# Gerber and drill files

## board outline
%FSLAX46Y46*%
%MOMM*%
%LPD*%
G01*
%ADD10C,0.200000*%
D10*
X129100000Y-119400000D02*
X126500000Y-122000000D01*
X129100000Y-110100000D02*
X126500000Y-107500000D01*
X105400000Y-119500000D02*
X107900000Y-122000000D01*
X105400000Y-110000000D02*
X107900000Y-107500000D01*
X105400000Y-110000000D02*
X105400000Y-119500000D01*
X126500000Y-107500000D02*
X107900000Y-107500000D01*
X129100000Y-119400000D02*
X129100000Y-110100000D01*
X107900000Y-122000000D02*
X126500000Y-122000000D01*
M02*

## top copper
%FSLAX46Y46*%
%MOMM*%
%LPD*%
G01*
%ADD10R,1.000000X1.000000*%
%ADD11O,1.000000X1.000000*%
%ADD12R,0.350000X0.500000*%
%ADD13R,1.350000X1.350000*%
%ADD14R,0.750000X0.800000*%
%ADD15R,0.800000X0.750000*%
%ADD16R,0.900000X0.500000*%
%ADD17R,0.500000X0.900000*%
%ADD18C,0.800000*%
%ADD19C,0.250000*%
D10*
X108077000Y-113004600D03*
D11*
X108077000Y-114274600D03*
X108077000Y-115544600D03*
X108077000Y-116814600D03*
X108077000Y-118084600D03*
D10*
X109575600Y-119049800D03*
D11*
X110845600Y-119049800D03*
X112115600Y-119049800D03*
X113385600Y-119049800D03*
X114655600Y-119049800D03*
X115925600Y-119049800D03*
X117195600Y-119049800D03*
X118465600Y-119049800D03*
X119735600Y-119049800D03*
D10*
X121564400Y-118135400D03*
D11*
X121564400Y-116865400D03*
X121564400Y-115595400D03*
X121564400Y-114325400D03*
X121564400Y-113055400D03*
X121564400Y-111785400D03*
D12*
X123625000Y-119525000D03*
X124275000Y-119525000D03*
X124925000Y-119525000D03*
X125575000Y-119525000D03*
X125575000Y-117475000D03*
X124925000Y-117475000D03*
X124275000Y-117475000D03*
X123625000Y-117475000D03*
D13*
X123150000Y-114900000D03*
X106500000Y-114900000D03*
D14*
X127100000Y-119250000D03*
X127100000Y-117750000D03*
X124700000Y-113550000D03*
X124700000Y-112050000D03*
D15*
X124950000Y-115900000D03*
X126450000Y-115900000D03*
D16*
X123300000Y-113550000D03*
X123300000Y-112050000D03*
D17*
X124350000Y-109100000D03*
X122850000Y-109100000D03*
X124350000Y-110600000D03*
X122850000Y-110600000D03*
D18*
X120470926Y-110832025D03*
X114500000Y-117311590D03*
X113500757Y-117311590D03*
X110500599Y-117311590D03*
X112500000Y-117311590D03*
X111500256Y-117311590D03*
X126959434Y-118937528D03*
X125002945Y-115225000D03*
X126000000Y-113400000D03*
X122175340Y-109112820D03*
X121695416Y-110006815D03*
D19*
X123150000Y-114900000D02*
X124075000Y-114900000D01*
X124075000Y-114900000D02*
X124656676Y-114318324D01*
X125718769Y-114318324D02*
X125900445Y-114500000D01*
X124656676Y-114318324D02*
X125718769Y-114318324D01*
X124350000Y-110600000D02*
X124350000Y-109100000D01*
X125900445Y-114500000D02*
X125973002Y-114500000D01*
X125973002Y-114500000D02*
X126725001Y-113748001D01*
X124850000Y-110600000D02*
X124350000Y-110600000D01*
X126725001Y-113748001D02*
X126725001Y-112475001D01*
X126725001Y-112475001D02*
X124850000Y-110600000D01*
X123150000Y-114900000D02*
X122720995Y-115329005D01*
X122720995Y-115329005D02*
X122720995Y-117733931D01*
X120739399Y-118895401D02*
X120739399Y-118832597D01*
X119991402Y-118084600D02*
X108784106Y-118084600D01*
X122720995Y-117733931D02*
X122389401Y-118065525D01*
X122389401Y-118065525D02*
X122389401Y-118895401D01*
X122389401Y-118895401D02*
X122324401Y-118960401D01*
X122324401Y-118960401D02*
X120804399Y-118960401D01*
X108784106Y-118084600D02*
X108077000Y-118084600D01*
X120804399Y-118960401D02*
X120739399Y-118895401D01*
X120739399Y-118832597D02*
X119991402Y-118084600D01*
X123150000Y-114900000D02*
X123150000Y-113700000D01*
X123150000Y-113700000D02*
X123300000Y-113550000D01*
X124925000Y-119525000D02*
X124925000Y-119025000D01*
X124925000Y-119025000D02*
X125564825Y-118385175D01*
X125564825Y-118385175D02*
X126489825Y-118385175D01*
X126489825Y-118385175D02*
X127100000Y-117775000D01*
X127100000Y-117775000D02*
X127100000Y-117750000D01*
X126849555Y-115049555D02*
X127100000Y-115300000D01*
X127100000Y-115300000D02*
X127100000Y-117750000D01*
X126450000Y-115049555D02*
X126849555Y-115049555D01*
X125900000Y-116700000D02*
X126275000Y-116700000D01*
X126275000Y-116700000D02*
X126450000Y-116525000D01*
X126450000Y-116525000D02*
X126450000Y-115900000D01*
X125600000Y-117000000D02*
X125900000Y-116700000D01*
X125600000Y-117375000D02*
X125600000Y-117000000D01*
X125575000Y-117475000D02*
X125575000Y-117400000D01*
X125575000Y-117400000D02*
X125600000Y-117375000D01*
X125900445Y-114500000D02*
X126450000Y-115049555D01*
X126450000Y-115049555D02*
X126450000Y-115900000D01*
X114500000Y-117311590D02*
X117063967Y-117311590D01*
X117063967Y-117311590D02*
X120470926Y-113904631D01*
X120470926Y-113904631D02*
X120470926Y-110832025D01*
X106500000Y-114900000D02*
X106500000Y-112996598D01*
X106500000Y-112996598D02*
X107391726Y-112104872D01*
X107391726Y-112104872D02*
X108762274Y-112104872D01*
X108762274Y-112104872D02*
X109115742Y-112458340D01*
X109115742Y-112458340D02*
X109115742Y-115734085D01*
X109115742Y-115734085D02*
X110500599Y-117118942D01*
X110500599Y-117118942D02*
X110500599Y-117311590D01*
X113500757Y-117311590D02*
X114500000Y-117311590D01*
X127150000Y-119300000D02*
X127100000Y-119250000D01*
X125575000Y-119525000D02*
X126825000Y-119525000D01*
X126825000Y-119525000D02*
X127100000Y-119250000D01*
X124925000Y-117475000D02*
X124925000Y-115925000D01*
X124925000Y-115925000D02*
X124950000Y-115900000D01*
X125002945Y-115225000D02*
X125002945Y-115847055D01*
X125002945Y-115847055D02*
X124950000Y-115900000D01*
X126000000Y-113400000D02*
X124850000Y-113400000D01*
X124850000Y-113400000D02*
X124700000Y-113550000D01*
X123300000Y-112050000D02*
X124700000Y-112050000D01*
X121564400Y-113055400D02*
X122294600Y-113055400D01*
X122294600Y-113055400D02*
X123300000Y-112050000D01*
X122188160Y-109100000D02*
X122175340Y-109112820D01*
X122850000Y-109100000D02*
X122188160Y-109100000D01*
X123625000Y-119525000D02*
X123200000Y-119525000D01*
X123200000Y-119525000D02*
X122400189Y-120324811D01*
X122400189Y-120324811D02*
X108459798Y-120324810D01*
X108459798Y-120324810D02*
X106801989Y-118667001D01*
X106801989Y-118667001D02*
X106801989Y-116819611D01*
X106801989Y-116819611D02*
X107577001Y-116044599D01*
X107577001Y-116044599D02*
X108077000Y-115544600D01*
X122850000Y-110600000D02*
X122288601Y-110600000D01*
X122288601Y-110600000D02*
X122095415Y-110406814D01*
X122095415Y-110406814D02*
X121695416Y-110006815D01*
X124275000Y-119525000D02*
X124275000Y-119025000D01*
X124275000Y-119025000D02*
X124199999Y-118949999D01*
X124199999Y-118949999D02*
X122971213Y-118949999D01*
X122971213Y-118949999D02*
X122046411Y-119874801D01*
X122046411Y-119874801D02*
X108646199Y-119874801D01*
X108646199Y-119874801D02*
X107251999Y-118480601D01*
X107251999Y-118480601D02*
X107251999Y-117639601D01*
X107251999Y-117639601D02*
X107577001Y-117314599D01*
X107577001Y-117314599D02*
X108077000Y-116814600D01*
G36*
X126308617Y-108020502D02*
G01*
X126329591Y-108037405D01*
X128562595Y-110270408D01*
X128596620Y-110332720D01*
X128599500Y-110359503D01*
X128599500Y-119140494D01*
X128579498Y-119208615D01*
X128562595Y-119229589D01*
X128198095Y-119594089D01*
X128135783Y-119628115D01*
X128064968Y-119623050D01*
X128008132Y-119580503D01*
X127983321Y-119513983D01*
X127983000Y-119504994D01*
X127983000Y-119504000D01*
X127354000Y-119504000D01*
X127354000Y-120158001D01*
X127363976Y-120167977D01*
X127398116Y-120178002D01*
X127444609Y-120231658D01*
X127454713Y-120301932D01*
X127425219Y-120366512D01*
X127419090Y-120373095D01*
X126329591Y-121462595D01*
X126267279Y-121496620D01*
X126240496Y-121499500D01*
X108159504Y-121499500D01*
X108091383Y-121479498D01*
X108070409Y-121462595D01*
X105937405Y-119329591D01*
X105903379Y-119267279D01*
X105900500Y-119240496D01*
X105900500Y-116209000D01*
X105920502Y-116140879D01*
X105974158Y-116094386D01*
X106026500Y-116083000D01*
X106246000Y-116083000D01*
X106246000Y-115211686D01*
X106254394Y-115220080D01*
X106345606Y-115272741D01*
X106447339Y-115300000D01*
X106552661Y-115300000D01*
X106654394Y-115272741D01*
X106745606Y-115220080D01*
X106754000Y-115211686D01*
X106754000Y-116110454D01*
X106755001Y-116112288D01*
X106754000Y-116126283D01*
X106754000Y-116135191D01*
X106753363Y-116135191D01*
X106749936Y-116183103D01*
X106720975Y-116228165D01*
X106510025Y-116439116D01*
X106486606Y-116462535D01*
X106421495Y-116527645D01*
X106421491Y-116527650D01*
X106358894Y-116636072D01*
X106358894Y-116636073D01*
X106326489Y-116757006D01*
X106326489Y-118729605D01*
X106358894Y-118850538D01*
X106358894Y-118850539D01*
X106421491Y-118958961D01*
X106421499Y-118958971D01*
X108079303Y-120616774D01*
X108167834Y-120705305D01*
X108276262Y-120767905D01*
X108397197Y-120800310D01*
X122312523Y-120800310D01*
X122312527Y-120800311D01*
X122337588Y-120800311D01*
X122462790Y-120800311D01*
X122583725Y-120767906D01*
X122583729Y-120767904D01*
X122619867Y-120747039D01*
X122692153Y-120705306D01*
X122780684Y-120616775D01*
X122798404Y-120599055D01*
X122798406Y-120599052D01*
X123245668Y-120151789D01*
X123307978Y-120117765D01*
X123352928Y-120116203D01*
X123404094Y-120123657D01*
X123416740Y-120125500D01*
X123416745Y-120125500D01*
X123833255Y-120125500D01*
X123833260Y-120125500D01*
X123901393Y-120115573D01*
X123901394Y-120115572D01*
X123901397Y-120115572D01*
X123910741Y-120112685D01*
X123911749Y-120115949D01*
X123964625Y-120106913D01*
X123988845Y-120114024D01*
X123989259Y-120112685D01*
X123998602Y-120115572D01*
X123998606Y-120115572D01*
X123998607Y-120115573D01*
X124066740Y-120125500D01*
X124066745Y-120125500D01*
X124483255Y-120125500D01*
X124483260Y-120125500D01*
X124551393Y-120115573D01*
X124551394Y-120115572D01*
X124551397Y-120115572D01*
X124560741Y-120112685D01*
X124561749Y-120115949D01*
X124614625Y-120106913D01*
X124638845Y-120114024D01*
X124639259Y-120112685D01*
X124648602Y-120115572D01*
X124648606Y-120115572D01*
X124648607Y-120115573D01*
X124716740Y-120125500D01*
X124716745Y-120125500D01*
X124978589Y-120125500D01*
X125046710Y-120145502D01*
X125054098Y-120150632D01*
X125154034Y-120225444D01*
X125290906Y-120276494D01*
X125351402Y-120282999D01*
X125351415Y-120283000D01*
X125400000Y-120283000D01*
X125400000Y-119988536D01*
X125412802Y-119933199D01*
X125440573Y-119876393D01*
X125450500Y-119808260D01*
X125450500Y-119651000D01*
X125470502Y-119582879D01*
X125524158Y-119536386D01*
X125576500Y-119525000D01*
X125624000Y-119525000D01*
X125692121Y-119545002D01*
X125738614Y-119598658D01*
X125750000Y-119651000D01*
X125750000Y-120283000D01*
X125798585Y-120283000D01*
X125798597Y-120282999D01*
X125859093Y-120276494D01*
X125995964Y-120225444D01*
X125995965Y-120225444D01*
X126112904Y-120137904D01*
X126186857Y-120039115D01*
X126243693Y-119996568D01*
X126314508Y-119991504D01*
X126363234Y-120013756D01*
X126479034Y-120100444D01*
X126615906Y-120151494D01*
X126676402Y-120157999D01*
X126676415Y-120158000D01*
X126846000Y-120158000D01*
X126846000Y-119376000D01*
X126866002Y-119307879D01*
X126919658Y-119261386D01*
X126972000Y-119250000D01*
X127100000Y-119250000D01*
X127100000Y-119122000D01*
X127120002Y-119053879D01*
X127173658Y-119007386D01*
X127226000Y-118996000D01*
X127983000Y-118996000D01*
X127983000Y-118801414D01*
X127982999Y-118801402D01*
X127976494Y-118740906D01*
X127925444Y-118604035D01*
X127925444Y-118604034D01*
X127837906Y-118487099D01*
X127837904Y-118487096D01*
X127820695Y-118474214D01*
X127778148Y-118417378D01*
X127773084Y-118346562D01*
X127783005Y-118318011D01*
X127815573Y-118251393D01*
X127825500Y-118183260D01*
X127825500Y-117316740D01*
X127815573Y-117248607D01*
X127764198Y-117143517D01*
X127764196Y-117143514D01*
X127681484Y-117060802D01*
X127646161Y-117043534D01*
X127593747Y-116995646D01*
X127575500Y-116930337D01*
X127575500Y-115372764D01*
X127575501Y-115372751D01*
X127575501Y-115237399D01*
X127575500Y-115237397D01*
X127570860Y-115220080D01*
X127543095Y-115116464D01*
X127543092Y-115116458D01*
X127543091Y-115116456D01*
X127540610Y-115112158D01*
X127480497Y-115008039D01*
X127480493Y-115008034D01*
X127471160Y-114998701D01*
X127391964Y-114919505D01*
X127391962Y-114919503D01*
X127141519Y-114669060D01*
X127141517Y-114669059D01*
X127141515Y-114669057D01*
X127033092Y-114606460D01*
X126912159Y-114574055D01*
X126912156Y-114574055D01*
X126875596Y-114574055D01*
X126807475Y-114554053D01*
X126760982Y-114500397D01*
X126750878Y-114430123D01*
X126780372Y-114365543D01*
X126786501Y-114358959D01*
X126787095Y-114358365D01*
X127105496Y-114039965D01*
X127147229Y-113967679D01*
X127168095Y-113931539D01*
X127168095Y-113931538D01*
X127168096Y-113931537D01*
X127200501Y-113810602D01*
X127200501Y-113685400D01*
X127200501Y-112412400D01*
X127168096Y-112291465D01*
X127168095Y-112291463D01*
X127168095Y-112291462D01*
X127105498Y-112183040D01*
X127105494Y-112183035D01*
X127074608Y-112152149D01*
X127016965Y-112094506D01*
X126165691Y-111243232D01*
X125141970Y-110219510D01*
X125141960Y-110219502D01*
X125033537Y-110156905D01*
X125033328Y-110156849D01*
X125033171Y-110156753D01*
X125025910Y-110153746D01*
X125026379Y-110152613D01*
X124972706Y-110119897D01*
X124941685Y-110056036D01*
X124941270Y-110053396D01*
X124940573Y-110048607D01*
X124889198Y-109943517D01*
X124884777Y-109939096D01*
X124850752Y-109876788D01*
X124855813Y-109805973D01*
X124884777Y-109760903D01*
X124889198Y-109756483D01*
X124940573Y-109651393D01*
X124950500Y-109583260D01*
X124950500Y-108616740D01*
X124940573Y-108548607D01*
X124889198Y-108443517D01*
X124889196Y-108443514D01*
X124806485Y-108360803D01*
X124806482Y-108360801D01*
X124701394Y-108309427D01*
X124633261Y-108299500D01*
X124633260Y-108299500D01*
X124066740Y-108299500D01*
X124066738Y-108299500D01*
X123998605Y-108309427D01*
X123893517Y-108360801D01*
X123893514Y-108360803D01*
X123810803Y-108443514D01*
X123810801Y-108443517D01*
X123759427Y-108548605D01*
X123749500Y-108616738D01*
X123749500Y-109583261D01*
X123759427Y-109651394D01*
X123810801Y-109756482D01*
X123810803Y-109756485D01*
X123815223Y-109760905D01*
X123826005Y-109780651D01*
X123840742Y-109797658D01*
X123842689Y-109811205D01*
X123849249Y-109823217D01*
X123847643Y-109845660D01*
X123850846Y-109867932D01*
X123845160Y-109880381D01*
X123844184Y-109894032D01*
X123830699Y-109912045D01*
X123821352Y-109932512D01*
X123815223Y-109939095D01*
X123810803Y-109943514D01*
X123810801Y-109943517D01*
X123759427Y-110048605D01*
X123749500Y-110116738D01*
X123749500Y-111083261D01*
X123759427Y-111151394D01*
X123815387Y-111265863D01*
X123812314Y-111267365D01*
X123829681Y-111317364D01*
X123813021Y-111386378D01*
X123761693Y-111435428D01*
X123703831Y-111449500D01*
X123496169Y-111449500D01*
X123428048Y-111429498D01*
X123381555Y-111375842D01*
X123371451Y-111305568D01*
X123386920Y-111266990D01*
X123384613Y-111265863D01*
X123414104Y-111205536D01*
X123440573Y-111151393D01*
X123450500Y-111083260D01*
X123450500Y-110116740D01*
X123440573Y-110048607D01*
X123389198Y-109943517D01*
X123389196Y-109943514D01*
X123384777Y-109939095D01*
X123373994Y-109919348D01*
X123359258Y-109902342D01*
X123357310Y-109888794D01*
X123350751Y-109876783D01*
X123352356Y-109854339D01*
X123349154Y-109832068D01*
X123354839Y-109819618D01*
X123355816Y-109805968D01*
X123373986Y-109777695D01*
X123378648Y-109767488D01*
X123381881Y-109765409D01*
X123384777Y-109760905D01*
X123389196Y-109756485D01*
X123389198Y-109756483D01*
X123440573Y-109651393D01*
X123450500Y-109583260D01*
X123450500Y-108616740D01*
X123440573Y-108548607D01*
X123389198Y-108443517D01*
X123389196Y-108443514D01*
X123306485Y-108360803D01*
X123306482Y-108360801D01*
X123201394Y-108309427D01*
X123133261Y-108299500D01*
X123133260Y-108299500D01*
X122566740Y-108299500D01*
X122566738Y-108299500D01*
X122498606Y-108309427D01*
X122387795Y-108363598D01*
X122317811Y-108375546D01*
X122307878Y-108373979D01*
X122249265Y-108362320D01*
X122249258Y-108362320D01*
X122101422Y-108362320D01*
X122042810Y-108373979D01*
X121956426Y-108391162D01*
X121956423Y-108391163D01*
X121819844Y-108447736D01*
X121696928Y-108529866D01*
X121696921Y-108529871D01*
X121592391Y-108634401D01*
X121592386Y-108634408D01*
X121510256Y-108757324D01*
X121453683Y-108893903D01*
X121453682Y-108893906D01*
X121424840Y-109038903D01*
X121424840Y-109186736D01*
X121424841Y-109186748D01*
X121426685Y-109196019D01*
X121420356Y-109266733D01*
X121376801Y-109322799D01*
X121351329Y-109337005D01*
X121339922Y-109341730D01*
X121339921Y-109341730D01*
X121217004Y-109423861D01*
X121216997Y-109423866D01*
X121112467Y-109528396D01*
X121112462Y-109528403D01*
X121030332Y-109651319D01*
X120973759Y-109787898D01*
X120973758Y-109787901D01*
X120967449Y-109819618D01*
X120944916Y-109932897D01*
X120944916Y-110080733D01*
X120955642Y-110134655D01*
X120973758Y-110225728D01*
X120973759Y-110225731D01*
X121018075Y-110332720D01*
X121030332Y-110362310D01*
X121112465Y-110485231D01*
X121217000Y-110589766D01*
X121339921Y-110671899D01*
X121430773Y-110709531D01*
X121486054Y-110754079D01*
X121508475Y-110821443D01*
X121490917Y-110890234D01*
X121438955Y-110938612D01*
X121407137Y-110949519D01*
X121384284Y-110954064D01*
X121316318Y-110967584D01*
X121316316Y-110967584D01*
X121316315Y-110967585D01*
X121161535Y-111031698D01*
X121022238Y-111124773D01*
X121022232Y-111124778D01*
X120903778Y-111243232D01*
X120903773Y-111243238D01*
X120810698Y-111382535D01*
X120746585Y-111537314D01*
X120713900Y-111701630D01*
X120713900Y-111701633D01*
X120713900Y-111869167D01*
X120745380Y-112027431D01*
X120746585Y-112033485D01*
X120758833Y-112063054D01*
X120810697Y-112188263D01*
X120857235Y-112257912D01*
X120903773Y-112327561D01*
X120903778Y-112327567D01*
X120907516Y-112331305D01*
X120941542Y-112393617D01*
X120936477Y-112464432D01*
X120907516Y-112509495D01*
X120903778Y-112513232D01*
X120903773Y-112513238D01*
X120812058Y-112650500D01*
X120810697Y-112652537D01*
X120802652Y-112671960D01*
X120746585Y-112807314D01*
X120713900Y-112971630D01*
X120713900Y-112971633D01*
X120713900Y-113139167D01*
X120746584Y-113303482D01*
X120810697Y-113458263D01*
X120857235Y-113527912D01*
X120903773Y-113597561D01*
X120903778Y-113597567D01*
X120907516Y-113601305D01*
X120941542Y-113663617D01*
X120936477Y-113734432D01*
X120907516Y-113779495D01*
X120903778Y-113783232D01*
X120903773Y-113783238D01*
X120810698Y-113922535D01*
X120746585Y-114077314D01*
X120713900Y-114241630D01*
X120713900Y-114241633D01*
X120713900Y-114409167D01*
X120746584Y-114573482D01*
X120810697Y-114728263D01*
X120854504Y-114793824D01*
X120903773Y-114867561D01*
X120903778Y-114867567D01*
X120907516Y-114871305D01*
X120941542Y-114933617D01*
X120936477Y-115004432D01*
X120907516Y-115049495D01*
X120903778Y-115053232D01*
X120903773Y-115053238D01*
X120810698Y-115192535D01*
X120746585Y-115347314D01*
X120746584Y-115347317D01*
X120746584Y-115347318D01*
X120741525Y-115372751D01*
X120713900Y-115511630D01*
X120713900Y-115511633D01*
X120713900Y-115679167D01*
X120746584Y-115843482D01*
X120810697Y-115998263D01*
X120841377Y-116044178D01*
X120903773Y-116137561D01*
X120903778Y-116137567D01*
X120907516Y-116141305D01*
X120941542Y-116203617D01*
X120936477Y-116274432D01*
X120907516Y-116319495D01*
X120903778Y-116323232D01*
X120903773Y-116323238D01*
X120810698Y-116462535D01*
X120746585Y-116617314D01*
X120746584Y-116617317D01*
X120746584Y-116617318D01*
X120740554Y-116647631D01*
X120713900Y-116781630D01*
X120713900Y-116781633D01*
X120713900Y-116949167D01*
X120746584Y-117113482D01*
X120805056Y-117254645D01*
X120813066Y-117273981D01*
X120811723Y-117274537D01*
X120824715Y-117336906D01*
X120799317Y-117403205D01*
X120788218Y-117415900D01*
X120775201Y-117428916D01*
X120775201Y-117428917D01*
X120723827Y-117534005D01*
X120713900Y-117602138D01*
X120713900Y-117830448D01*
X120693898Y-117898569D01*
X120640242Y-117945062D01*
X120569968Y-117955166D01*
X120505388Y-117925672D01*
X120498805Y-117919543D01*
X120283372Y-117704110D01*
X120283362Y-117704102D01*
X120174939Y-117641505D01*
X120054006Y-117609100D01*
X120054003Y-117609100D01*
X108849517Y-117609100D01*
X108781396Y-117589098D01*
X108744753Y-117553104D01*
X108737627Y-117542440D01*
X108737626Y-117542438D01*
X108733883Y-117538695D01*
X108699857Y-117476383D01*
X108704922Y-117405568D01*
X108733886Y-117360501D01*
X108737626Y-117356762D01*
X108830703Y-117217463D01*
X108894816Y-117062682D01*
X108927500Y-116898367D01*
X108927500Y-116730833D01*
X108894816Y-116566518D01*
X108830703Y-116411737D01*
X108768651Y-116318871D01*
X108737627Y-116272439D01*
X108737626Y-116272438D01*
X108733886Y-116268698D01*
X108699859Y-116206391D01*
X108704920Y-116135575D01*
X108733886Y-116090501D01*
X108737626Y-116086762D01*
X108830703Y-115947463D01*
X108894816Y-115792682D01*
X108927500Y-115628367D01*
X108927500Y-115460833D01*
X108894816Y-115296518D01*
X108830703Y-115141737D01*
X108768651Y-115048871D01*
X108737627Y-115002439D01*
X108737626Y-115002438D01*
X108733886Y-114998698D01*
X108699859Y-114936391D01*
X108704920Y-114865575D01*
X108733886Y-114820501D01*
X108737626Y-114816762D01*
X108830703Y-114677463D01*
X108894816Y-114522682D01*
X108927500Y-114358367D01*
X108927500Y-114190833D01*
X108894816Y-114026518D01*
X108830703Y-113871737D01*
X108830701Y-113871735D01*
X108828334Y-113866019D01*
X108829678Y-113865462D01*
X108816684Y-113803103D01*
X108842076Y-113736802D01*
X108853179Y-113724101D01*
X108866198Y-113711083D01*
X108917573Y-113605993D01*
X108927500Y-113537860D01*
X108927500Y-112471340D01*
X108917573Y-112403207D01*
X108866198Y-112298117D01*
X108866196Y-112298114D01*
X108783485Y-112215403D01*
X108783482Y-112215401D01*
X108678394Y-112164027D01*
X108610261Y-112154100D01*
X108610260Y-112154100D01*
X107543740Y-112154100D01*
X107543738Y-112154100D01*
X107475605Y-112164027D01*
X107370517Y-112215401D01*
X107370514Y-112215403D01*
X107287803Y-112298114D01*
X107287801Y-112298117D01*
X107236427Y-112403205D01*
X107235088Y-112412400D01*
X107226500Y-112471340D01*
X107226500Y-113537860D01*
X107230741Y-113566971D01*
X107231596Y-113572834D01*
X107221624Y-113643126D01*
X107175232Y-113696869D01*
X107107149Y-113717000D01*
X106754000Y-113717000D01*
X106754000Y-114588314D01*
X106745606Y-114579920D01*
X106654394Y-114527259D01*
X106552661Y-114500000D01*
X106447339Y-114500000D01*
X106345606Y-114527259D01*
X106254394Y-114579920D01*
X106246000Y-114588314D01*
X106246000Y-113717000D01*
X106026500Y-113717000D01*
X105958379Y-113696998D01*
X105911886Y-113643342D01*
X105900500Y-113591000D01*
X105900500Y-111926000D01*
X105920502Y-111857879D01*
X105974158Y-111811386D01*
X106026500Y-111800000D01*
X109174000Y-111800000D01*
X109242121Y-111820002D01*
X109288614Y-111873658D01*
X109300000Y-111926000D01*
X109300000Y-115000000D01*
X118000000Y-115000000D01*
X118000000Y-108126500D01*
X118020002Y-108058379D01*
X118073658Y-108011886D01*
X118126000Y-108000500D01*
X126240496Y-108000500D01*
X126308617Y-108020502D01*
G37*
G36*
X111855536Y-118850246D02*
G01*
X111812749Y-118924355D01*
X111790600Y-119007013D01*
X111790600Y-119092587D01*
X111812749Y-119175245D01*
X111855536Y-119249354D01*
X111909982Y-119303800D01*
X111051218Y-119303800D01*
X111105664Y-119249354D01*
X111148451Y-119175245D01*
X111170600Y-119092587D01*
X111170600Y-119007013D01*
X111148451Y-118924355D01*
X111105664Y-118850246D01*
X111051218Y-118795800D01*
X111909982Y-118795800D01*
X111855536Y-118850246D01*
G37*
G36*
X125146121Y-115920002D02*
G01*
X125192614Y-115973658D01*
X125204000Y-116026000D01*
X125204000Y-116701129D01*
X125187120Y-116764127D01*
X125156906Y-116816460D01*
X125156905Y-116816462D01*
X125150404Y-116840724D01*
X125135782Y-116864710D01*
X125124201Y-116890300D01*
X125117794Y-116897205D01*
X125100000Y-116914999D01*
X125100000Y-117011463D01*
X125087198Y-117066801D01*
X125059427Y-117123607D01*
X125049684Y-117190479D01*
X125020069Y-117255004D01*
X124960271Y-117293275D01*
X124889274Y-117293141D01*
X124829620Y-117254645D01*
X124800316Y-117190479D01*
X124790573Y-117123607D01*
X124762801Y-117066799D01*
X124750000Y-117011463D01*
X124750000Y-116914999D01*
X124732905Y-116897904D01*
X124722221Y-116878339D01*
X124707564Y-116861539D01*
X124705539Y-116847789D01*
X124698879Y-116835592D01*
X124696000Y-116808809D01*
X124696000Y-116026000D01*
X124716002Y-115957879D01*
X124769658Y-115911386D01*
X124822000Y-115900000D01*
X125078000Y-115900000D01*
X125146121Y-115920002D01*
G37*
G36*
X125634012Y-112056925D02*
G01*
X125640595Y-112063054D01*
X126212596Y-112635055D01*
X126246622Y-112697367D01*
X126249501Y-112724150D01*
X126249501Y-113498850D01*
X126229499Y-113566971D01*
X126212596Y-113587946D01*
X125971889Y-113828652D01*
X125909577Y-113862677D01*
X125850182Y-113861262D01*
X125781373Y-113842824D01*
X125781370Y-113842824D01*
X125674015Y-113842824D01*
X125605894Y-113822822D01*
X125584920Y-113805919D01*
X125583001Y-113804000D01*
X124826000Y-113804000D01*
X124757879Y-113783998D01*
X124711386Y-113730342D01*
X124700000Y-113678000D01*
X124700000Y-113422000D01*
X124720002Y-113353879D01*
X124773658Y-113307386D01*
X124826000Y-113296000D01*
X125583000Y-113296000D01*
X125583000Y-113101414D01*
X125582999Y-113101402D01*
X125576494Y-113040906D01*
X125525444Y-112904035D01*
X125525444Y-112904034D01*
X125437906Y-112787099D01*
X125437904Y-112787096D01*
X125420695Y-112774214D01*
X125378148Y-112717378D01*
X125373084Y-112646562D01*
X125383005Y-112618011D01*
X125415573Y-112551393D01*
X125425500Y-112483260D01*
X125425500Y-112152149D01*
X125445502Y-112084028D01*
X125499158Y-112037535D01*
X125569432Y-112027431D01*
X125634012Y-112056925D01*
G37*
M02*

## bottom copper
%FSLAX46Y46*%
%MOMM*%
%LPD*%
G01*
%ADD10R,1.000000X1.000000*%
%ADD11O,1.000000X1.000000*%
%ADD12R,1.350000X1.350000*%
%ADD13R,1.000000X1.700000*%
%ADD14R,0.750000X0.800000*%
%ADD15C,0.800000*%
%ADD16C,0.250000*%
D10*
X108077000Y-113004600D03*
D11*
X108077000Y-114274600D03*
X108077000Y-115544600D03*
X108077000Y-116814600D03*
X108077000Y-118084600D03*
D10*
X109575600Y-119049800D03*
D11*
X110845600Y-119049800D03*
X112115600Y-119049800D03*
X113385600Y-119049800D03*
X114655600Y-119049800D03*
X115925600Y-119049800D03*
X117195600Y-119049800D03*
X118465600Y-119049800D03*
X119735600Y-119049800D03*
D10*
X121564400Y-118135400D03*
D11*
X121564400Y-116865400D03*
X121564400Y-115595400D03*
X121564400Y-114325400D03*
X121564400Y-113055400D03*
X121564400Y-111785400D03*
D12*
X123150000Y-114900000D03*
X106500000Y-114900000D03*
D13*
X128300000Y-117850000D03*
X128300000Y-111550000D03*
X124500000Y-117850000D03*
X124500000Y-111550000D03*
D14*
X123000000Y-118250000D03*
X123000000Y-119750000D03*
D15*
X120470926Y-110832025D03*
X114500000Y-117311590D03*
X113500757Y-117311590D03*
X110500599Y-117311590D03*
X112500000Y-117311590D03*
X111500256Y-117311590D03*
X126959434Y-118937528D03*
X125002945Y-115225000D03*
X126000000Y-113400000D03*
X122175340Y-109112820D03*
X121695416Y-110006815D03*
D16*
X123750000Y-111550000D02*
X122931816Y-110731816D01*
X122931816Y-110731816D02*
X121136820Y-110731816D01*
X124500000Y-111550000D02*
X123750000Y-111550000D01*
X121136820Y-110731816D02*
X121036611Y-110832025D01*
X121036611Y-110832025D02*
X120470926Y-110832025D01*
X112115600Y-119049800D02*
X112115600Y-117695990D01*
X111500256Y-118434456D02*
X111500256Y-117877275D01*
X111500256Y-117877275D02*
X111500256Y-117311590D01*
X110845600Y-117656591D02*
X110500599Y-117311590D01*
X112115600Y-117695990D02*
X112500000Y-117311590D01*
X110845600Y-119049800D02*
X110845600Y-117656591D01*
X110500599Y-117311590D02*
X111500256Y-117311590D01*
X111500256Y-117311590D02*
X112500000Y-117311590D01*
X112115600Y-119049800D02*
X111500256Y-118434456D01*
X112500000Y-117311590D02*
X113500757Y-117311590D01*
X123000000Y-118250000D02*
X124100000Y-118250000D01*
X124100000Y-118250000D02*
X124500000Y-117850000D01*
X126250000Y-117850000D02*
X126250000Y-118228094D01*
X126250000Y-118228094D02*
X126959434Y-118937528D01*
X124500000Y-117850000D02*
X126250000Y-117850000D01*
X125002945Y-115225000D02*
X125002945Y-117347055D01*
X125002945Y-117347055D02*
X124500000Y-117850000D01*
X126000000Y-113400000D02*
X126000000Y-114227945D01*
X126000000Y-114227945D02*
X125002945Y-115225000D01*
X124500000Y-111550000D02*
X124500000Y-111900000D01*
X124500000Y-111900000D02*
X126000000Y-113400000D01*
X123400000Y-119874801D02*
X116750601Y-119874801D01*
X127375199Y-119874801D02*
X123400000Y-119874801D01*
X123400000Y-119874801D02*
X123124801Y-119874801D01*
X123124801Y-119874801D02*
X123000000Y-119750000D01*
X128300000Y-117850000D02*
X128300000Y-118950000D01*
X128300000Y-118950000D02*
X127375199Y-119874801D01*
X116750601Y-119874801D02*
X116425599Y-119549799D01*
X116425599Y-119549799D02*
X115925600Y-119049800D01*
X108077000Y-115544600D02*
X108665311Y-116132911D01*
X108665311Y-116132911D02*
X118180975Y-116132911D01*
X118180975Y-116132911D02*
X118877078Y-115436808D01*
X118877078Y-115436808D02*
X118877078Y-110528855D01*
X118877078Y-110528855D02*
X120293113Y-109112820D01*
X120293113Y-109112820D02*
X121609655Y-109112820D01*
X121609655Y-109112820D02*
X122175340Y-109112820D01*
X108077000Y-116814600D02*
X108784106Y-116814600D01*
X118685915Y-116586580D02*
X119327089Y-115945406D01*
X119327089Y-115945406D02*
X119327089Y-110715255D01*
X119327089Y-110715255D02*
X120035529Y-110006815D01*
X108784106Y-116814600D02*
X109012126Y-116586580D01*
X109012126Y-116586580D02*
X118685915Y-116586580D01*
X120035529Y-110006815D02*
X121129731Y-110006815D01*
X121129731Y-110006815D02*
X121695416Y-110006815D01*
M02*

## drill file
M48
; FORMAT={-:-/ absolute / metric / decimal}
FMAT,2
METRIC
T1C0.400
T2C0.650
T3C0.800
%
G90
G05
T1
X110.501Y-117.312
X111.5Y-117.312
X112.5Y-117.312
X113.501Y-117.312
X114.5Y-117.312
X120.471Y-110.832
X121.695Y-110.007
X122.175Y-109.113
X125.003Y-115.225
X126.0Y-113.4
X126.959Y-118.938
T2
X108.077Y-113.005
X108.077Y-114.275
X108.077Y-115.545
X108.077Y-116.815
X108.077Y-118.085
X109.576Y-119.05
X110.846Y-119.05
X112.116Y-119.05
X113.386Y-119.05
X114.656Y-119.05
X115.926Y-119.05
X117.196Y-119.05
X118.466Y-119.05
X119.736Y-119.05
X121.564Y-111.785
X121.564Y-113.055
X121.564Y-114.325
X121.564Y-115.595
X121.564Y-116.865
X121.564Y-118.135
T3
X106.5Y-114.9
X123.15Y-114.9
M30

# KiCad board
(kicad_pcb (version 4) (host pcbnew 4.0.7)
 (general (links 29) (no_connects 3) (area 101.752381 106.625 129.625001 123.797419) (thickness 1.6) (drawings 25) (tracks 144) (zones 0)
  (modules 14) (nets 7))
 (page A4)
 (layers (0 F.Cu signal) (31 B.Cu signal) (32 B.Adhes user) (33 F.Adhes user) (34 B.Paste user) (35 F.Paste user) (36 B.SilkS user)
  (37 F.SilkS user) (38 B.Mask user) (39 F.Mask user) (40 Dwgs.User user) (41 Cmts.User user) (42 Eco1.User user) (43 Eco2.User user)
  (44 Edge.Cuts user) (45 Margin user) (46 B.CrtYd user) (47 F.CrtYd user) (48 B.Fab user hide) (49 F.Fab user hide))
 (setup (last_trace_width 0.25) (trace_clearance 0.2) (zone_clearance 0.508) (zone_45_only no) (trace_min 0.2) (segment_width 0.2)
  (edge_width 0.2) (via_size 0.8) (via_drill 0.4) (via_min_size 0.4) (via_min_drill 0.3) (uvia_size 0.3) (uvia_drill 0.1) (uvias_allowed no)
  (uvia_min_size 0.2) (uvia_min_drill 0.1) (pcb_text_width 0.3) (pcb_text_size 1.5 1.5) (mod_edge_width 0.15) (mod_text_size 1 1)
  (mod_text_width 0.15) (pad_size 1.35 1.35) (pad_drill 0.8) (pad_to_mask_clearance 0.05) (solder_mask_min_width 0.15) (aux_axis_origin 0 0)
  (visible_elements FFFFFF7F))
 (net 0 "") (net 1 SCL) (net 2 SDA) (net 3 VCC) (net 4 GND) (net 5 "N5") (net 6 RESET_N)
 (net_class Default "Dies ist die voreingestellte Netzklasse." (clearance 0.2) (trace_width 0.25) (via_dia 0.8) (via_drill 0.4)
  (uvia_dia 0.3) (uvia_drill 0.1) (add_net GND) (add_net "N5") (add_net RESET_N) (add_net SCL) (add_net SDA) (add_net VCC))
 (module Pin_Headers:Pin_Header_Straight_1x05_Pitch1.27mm (layer F.Cu) (at 108.077 113.0046)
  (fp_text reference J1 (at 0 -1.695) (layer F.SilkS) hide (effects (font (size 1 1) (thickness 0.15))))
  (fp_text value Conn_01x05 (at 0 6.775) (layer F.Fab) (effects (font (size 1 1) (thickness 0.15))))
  (pad 1 thru_hole rect (at 0 0) (size 1 1) (drill 0.65) (layers *.Cu *.Mask))
  (pad 2 thru_hole oval (at 0 1.27) (size 1 1) (drill 0.65) (layers *.Cu *.Mask))
  (pad 3 thru_hole oval (at 0 2.54) (size 1 1) (drill 0.65) (layers *.Cu *.Mask) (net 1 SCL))
  (pad 4 thru_hole oval (at 0 3.81) (size 1 1) (drill 0.65) (layers *.Cu *.Mask) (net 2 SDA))
  (pad 5 thru_hole oval (at 0 5.08) (size 1 1) (drill 0.65) (layers *.Cu *.Mask) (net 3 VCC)))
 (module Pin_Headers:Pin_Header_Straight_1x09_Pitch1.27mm (layer F.Cu) (at 109.5756 119.0498 90)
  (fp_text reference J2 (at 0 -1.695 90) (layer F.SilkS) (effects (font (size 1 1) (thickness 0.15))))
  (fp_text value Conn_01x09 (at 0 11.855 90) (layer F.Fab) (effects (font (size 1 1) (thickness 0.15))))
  (pad 1 thru_hole rect (at 0 0 90) (size 1 1) (drill 0.65) (layers *.Cu *.Mask))
  (pad 2 thru_hole oval (at 0 1.27 90) (size 1 1) (drill 0.65) (layers *.Cu *.Mask) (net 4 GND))
  (pad 3 thru_hole oval (at 0 2.54 90) (size 1 1) (drill 0.65) (layers *.Cu *.Mask) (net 4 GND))
  (pad 4 thru_hole oval (at 0 3.81 90) (size 1 1) (drill 0.65) (layers *.Cu *.Mask))
  (pad 5 thru_hole oval (at 0 5.08 90) (size 1 1) (drill 0.65) (layers *.Cu *.Mask))
  (pad 6 thru_hole oval (at 0 6.35 90) (size 1 1) (drill 0.65) (layers *.Cu *.Mask) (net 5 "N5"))
  (pad 7 thru_hole oval (at 0 7.62 90) (size 1 1) (drill 0.65) (layers *.Cu *.Mask))
  (pad 8 thru_hole oval (at 0 8.89 90) (size 1 1) (drill 0.65) (layers *.Cu *.Mask))
  (pad 9 thru_hole oval (at 0 10.16 90) (size 1 1) (drill 0.65) (layers *.Cu *.Mask)))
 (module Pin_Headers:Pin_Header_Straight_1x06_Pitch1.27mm (layer F.Cu) (at 121.5644 118.1354 180)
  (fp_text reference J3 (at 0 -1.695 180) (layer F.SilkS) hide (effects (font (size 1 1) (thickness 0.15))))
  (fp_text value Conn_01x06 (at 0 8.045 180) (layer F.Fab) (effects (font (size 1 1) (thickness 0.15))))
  (pad 1 thru_hole rect (at 0 0 180) (size 1 1) (drill 0.65) (layers *.Cu *.Mask))
  (pad 2 thru_hole oval (at 0 1.27 180) (size 1 1) (drill 0.65) (layers *.Cu *.Mask))
  (pad 3 thru_hole oval (at 0 2.54 180) (size 1 1) (drill 0.65) (layers *.Cu *.Mask))
  (pad 4 thru_hole oval (at 0 3.81 180) (size 1 1) (drill 0.65) (layers *.Cu *.Mask))
  (pad 5 thru_hole oval (at 0 5.08 180) (size 1 1) (drill 0.65) (layers *.Cu *.Mask) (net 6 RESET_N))
  (pad 6 thru_hole oval (at 0 6.35 180) (size 1 1) (drill 0.65) (layers *.Cu *.Mask)))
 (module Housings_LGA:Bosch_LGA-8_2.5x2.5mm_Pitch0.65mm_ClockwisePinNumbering (layer F.Cu) (at 124.6 118.5 180)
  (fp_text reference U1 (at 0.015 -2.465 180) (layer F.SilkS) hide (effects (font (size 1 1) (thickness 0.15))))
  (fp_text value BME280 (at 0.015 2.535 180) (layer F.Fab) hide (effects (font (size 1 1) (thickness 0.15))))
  (pad 4 smd rect (at 0.975 -1.025 270) (size 0.5 0.35) (layers F.Cu F.Paste F.Mask) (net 1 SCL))
  (pad 3 smd rect (at 0.325 -1.025 270) (size 0.5 0.35) (layers F.Cu F.Paste F.Mask) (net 2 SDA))
  (pad 2 smd rect (at -0.325 -1.025 270) (size 0.5 0.35) (layers F.Cu F.Paste F.Mask) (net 3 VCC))
  (pad 1 smd rect (at -0.975 -1.025 270) (size 0.5 0.35) (layers F.Cu F.Paste F.Mask) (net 4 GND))
  (pad 8 smd rect (at -0.975 1.025 270) (size 0.5 0.35) (layers F.Cu F.Paste F.Mask) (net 3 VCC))
  (pad 7 smd rect (at -0.325 1.025 270) (size 0.5 0.35) (layers F.Cu F.Paste F.Mask) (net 4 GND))
  (pad 6 smd rect (at 0.325 1.025 270) (size 0.5 0.35) (layers F.Cu F.Paste F.Mask) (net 3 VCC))
  (pad 5 smd rect (at 0.975 1.025 270) (size 0.5 0.35) (layers F.Cu F.Paste F.Mask) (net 3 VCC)))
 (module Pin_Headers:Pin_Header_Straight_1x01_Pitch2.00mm (layer F.Cu) (at 123.15 114.7)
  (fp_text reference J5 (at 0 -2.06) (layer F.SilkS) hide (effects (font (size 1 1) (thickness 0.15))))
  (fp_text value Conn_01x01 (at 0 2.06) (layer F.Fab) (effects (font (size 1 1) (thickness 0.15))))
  (pad 1 thru_hole rect (at 0 0.2) (size 1.35 1.35) (drill 0.8) (layers *.Cu *.Mask) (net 3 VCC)))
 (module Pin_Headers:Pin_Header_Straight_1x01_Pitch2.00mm (layer F.Cu) (at 106.5 114.8)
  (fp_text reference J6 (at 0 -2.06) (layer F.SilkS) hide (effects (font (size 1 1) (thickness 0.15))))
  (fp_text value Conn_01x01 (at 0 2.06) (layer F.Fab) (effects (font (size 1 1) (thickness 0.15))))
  (pad 1 thru_hole rect (at 0 0.1) (size 1.35 1.35) (drill 0.8) (layers *.Cu *.Mask) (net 4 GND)))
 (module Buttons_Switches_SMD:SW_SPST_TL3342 (layer B.Cu) (at 126.4 114.7 90)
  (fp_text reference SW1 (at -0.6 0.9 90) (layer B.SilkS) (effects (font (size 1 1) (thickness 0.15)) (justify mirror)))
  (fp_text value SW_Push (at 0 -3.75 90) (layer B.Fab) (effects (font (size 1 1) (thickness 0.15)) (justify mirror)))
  (pad 1 smd rect (at -3.15 1.9 90) (size 1.7 1) (layers B.Cu B.Paste B.Mask) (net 5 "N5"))
  (pad 1 smd rect (at 3.15 1.9 90) (size 1.7 1) (layers B.Cu B.Paste B.Mask) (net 5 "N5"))
  (pad 2 smd rect (at -3.15 -1.9 90) (size 1.7 1) (layers B.Cu B.Paste B.Mask) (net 4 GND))
  (pad 2 smd rect (at 3.15 -1.9 90) (size 1.7 1) (layers B.Cu B.Paste B.Mask) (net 4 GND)))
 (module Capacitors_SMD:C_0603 (layer F.Cu) (at 127.1 118.5 270)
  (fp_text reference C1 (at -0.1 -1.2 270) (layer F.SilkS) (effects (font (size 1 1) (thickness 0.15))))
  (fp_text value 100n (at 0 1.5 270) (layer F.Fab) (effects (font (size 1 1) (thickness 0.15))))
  (pad 2 smd rect (at 0.75 0 270) (size 0.8 0.75) (layers F.Cu F.Paste F.Mask) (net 4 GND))
  (pad 1 smd rect (at -0.75 0 270) (size 0.8 0.75) (layers F.Cu F.Paste F.Mask) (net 3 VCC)))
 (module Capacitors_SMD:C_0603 (layer F.Cu) (at 124.7 112.8 270)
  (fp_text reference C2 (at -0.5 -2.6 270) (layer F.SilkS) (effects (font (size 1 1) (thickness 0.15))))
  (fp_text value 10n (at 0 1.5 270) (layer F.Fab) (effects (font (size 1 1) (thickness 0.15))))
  (pad 2 smd rect (at 0.75 0 270) (size 0.8 0.75) (layers F.Cu F.Paste F.Mask) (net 4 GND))
  (pad 1 smd rect (at -0.75 0 270) (size 0.8 0.75) (layers F.Cu F.Paste F.Mask) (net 6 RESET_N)))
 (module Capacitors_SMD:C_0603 (layer F.Cu) (at 125.7 115.9 180)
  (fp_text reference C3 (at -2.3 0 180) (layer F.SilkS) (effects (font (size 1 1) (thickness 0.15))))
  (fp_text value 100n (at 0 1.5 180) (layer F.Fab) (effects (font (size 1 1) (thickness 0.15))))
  (pad 2 smd rect (at 0.75 0 180) (size 0.8 0.75) (layers F.Cu F.Paste F.Mask) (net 4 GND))
  (pad 1 smd rect (at -0.75 0 180) (size 0.8 0.75) (layers F.Cu F.Paste F.Mask) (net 3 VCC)))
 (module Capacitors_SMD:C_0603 (layer B.Cu) (at 123 119 90)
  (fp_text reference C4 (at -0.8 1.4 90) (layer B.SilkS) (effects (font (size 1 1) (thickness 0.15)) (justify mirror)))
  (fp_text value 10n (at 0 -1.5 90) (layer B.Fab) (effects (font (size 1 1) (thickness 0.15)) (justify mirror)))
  (pad 2 smd rect (at 0.75 0 90) (size 0.8 0.75) (layers B.Cu B.Paste B.Mask) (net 4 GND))
  (pad 1 smd rect (at -0.75 0 90) (size 0.8 0.75) (layers B.Cu B.Paste B.Mask) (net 5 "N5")))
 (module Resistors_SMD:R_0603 (layer F.Cu) (at 123.3 112.8 90)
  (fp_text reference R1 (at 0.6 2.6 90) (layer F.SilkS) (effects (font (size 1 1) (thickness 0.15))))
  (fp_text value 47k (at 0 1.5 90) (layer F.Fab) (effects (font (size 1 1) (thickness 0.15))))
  (pad 1 smd rect (at -0.75 0 90) (size 0.5 0.9) (layers F.Cu F.Paste F.Mask) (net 3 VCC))
  (pad 2 smd rect (at 0.75 0 90) (size 0.5 0.9) (layers F.Cu F.Paste F.Mask) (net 6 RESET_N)))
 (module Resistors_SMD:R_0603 (layer F.Cu) (at 123.6 109.1 180)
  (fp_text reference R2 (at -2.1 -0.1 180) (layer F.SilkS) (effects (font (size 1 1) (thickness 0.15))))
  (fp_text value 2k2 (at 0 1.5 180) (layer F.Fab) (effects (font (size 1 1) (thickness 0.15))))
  (pad 1 smd rect (at -0.75 0 180) (size 0.5 0.9) (layers F.Cu F.Paste F.Mask) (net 3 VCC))
  (pad 2 smd rect (at 0.75 0 180) (size 0.5 0.9) (layers F.Cu F.Paste F.Mask) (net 1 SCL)))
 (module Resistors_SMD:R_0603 (layer F.Cu) (at 123.6 110.6 180)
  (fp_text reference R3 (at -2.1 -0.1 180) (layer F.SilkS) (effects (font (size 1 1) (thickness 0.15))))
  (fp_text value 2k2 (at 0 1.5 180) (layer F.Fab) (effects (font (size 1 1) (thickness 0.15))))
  (pad 1 smd rect (at -0.75 0 180) (size 0.5 0.9) (layers F.Cu F.Paste F.Mask) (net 3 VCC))
  (pad 2 smd rect (at 0.75 0 180) (size 0.5 0.9) (layers F.Cu F.Paste F.Mask) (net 2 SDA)))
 (gr_line (start 129.1 119.4) (end 126.5 122) (layer Edge.Cuts) (width 0.2))
 (gr_line (start 129.1 110.1) (end 126.5 107.5) (layer Edge.Cuts) (width 0.2))
 (gr_line (start 105.4 119.5) (end 107.9 122) (layer Edge.Cuts) (width 0.2))
 (gr_line (start 105.4 110) (end 107.9 107.5) (layer Edge.Cuts) (width 0.2))
 (gr_line (start 105.4 110) (end 105.4 119.5) (layer Edge.Cuts) (width 0.2))
 (gr_line (start 126.5 107.5) (end 107.9 107.5) (layer Edge.Cuts) (width 0.2))
 (gr_line (start 129.1 119.4) (end 129.1 110.1) (layer Edge.Cuts) (width 0.2))
 (gr_line (start 107.9 122) (end 126.5 122) (layer Edge.Cuts) (width 0.2))
 (segment (start 123.15 114.9) (end 124.075 114.9) (width 0.25) (layer F.Cu) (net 3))
 (segment (start 124.075 114.9) (end 124.656676 114.318324) (width 0.25) (layer F.Cu) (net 3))
 (segment (start 125.718769 114.318324) (end 125.900445 114.5) (width 0.25) (layer F.Cu) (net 3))
 (segment (start 124.656676 114.318324) (end 125.718769 114.318324) (width 0.25) (layer F.Cu) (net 3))
 (segment (start 124.35 110.6) (end 124.35 109.1) (width 0.25) (layer F.Cu) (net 3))
 (segment (start 125.900445 114.5) (end 125.973002 114.5) (width 0.25) (layer F.Cu) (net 3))
 (segment (start 125.973002 114.5) (end 126.725001 113.748001) (width 0.25) (layer F.Cu) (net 3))
 (segment (start 124.85 110.6) (end 124.35 110.6) (width 0.25) (layer F.Cu) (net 3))
 (segment (start 126.725001 113.748001) (end 126.725001 112.475001) (width 0.25) (layer F.Cu) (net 3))
 (segment (start 126.725001 112.475001) (end 124.85 110.6) (width 0.25) (layer F.Cu) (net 3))
 (segment (start 123.15 114.9) (end 122.720995 115.329005) (width 0.25) (layer F.Cu) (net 3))
 (segment (start 122.720995 115.329005) (end 122.720995 117.733931) (width 0.25) (layer F.Cu) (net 3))
 (segment (start 120.739399 118.895401) (end 120.739399 118.832597) (width 0.25) (layer F.Cu) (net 3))
 (segment (start 119.991402 118.0846) (end 108.784106 118.0846) (width 0.25) (layer F.Cu) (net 3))
 (segment (start 122.720995 117.733931) (end 122.389401 118.065525) (width 0.25) (layer F.Cu) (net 3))
 (segment (start 122.389401 118.065525) (end 122.389401 118.895401) (width 0.25) (layer F.Cu) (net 3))
 (segment (start 122.389401 118.895401) (end 122.324401 118.960401) (width 0.25) (layer F.Cu) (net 3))
 (segment (start 122.324401 118.960401) (end 120.804399 118.960401) (width 0.25) (layer F.Cu) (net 3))
 (segment (start 108.784106 118.0846) (end 108.077 118.0846) (width 0.25) (layer F.Cu) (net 3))
 (segment (start 120.804399 118.960401) (end 120.739399 118.895401) (width 0.25) (layer F.Cu) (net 3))
 (segment (start 120.739399 118.832597) (end 119.991402 118.0846) (width 0.25) (layer F.Cu) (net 3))
 (segment (start 123.15 114.9) (end 123.15 113.7) (width 0.25) (layer F.Cu) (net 3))
 (segment (start 123.15 113.7) (end 123.3 113.55) (width 0.25) (layer F.Cu) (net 3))
 (segment (start 124.925 119.525) (end 124.925 119.025) (width 0.25) (layer F.Cu) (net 3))
 (segment (start 124.925 119.025) (end 125.564825 118.385175) (width 0.25) (layer F.Cu) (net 3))
 (segment (start 125.564825 118.385175) (end 126.489825 118.385175) (width 0.25) (layer F.Cu) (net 3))
 (segment (start 126.489825 118.385175) (end 127.1 117.775) (width 0.25) (layer F.Cu) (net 3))
 (segment (start 127.1 117.775) (end 127.1 117.75) (width 0.25) (layer F.Cu) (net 3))
 (segment (start 126.849555 115.049555) (end 127.1 115.3) (width 0.25) (layer F.Cu) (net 3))
 (segment (start 127.1 115.3) (end 127.1 117.75) (width 0.25) (layer F.Cu) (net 3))
 (segment (start 126.45 115.049555) (end 126.849555 115.049555) (width 0.25) (layer F.Cu) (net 3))
 (segment (start 125.9 116.7) (end 126.275 116.7) (width 0.25) (layer F.Cu) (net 3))
 (segment (start 126.275 116.7) (end 126.45 116.525) (width 0.25) (layer F.Cu) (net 3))
 (segment (start 126.45 116.525) (end 126.45 115.9) (width 0.25) (layer F.Cu) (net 3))
 (segment (start 125.6 117) (end 125.9 116.7) (width 0.25) (layer F.Cu) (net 3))
 (segment (start 125.6 117.375) (end 125.6 117) (width 0.25) (layer F.Cu) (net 3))
 (segment (start 125.575 117.475) (end 125.575 117.4) (width 0.25) (layer F.Cu) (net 3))
 (segment (start 125.575 117.4) (end 125.6 117.375) (width 0.25) (layer F.Cu) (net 3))
 (segment (start 125.900445 114.5) (end 126.45 115.049555) (width 0.25) (layer F.Cu) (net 3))
 (segment (start 126.45 115.049555) (end 126.45 115.9) (width 0.25) (layer F.Cu) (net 3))
 (segment (start 114.5 117.31159) (end 117.063967 117.31159) (width 0.25) (layer F.Cu) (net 4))
 (segment (start 117.063967 117.31159) (end 120.470926 113.904631) (width 0.25) (layer F.Cu) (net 4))
 (segment (start 120.470926 113.904631) (end 120.470926 110.832025) (width 0.25) (layer F.Cu) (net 4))
 (via (at 120.470926 110.832025) (size 0.8) (drill 0.4) (layers F.Cu B.Cu) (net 4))
 (segment (start 123.75 111.55) (end 122.931816 110.731816) (width 0.25) (layer B.Cu) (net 4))
 (segment (start 122.931816 110.731816) (end 121.13682 110.731816) (width 0.25) (layer B.Cu) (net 4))
 (segment (start 124.5 111.55) (end 123.75 111.55) (width 0.25) (layer B.Cu) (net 4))
 (segment (start 121.13682 110.731816) (end 121.036611 110.832025) (width 0.25) (layer B.Cu) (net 4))
 (segment (start 121.036611 110.832025) (end 120.470926 110.832025) (width 0.25) (layer B.Cu) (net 4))
 (segment (start 106.5 114.9) (end 106.5 112.996598) (width 0.25) (layer F.Cu) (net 4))
 (segment (start 106.5 112.996598) (end 107.391726 112.104872) (width 0.25) (layer F.Cu) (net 4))
 (segment (start 107.391726 112.104872) (end 108.762274 112.104872) (width 0.25) (layer F.Cu) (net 4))
 (segment (start 108.762274 112.104872) (end 109.115742 112.45834) (width 0.25) (layer F.Cu) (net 4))
 (segment (start 109.115742 112.45834) (end 109.115742 115.734085) (width 0.25) (layer F.Cu) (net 4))
 (segment (start 109.115742 115.734085) (end 110.500599 117.118942) (width 0.25) (layer F.Cu) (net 4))
 (segment (start 110.500599 117.118942) (end 110.500599 117.31159) (width 0.25) (layer F.Cu) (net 4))
 (segment (start 113.500757 117.31159) (end 114.5 117.31159) (width 0.25) (layer F.Cu) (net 4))
 (via (at 114.5 117.31159) (size 0.8) (drill 0.4) (layers F.Cu B.Cu) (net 4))
 (segment (start 112.1156 119.0498) (end 112.1156 117.69599) (width 0.25) (layer B.Cu) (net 4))
 (segment (start 111.500256 118.434456) (end 111.500256 117.877275) (width 0.25) (layer B.Cu) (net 4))
 (segment (start 111.500256 117.877275) (end 111.500256 117.31159) (width 0.25) (layer B.Cu) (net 4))
 (segment (start 110.8456 117.656591) (end 110.500599 117.31159) (width 0.25) (layer B.Cu) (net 4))
 (via (at 113.500757 117.31159) (size 0.8) (drill 0.4) (layers F.Cu B.Cu) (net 4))
 (segment (start 112.1156 117.69599) (end 112.5 117.31159) (width 0.25) (layer B.Cu) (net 4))
 (via (at 110.500599 117.31159) (size 0.8) (drill 0.4) (layers F.Cu B.Cu) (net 4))
 (via (at 112.5 117.31159) (size 0.8) (drill 0.4) (layers F.Cu B.Cu) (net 4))
 (segment (start 110.8456 119.0498) (end 110.8456 117.656591) (width 0.25) (layer B.Cu) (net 4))
 (segment (start 110.500599 117.31159) (end 111.500256 117.31159) (width 0.25) (layer B.Cu) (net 4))
 (via (at 111.500256 117.31159) (size 0.8) (drill 0.4) (layers F.Cu B.Cu) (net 4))
 (segment (start 111.500256 117.31159) (end 112.5 117.31159) (width 0.25) (layer B.Cu) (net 4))
 (segment (start 112.1156 119.0498) (end 111.500256 118.434456) (width 0.25) (layer B.Cu) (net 4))
 (segment (start 112.5 117.31159) (end 113.500757 117.31159) (width 0.25) (layer B.Cu) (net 4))
 (segment (start 123 118.25) (end 124.1 118.25) (width 0.25) (layer B.Cu) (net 4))
 (segment (start 124.1 118.25) (end 124.5 117.85) (width 0.25) (layer B.Cu) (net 4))
 (segment (start 126.25 117.85) (end 126.25 118.228094) (width 0.25) (layer B.Cu) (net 4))
 (segment (start 126.25 118.228094) (end 126.959434 118.937528) (width 0.25) (layer B.Cu) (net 4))
 (via (at 126.959434 118.937528) (size 0.8) (drill 0.4) (layers F.Cu B.Cu) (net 4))
 (segment (start 127.15 119.3) (end 127.1 119.25) (width 0.25) (layer F.Cu) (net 4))
 (segment (start 124.5 117.85) (end 126.25 117.85) (width 0.25) (layer B.Cu) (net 4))
 (segment (start 125.002945 115.225) (end 125.002945 117.347055) (width 0.25) (layer B.Cu) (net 4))
 (segment (start 125.002945 117.347055) (end 124.5 117.85) (width 0.25) (layer B.Cu) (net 4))
 (segment (start 125.575 119.525) (end 126.825 119.525) (width 0.25) (layer F.Cu) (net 4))
 (segment (start 126.825 119.525) (end 127.1 119.25) (width 0.25) (layer F.Cu) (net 4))
 (segment (start 124.925 117.475) (end 124.925 115.925) (width 0.25) (layer F.Cu) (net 4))
 (segment (start 124.925 115.925) (end 124.95 115.9) (width 0.25) (layer F.Cu) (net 4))
 (segment (start 125.002945 115.225) (end 125.002945 115.847055) (width 0.25) (layer F.Cu) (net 4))
 (segment (start 125.002945 115.847055) (end 124.95 115.9) (width 0.25) (layer F.Cu) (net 4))
 (segment (start 126 113.4) (end 126 114.227945) (width 0.25) (layer B.Cu) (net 4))
 (segment (start 126 114.227945) (end 125.002945 115.225) (width 0.25) (layer B.Cu) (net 4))
 (via (at 125.002945 115.225) (size 0.8) (drill 0.4) (layers F.Cu B.Cu) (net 4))
 (segment (start 126 113.4) (end 124.85 113.4) (width 0.25) (layer F.Cu) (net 4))
 (segment (start 124.85 113.4) (end 124.7 113.55) (width 0.25) (layer F.Cu) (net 4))
 (segment (start 124.5 111.55) (end 124.5 111.9) (width 0.25) (layer B.Cu) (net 4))
 (segment (start 124.5 111.9) (end 126 113.4) (width 0.25) (layer B.Cu) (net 4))
 (via (at 126 113.4) (size 0.8) (drill 0.4) (layers F.Cu B.Cu) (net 4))
 (segment (start 123.3 112.05) (end 124.7 112.05) (width 0.25) (layer F.Cu) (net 6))
 (segment (start 121.5644 113.0554) (end 122.2946 113.0554) (width 0.25) (layer F.Cu) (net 6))
 (segment (start 122.2946 113.0554) (end 123.3 112.05) (width 0.25) (layer F.Cu) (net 6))
 (segment (start 123.4 119.874801) (end 116.750601 119.874801) (width 0.25) (layer B.Cu) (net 5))
 (segment (start 127.375199 119.874801) (end 123.4 119.874801) (width 0.25) (layer B.Cu) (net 5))
 (segment (start 123.4 119.874801) (end 123.124801 119.874801) (width 0.25) (layer B.Cu) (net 5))
 (segment (start 123.124801 119.874801) (end 123 119.75) (width 0.25) (layer B.Cu) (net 5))
 (segment (start 128.3 117.85) (end 128.3 118.95) (width 0.25) (layer B.Cu) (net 5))
 (segment (start 128.3 118.95) (end 127.375199 119.874801) (width 0.25) (layer B.Cu) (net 5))
 (segment (start 116.750601 119.874801) (end 116.425599 119.549799) (width 0.25) (layer B.Cu) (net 5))
 (segment (start 116.425599 119.549799) (end 115.9256 119.0498) (width 0.25) (layer B.Cu) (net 5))
 (segment (start 108.077 115.5446) (end 108.665311 116.132911) (width 0.25) (layer B.Cu) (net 1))
 (segment (start 108.665311 116.132911) (end 118.180975 116.132911) (width 0.25) (layer B.Cu) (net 1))
 (segment (start 118.180975 116.132911) (end 118.877078 115.436808) (width 0.25) (layer B.Cu) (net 1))
 (segment (start 118.877078 115.436808) (end 118.877078 110.528855) (width 0.25) (layer B.Cu) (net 1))
 (segment (start 118.877078 110.528855) (end 120.293113 109.11282) (width 0.25) (layer B.Cu) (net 1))
 (segment (start 120.293113 109.11282) (end 121.609655 109.11282) (width 0.25) (layer B.Cu) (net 1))
 (segment (start 121.609655 109.11282) (end 122.17534 109.11282) (width 0.25) (layer B.Cu) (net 1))
 (segment (start 122.18816 109.1) (end 122.17534 109.11282) (width 0.25) (layer F.Cu) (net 1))
 (segment (start 122.85 109.1) (end 122.18816 109.1) (width 0.25) (layer F.Cu) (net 1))
 (via (at 122.17534 109.11282) (size 0.8) (drill 0.4) (layers F.Cu B.Cu) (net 1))
 (segment (start 123.625 119.525) (end 123.2 119.525) (width 0.25) (layer F.Cu) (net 1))
 (segment (start 123.2 119.525) (end 122.400189 120.324811) (width 0.25) (layer F.Cu) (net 1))
 (segment (start 122.400189 120.324811) (end 108.459798 120.32481) (width 0.25) (layer F.Cu) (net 1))
 (segment (start 108.459798 120.32481) (end 106.801989 118.667001) (width 0.25) (layer F.Cu) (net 1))
 (segment (start 106.801989 118.667001) (end 106.801989 116.819611) (width 0.25) (layer F.Cu) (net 1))
 (segment (start 106.801989 116.819611) (end 107.577001 116.044599) (width 0.25) (layer F.Cu) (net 1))
 (segment (start 107.577001 116.044599) (end 108.077 115.5446) (width 0.25) (layer F.Cu) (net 1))
 (segment (start 108.077 116.8146) (end 108.784106 116.8146) (width 0.25) (layer B.Cu) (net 2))
 (segment (start 118.685915 116.58658) (end 119.327089 115.945406) (width 0.25) (layer B.Cu) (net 2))
 (segment (start 119.327089 115.945406) (end 119.327089 110.715255) (width 0.25) (layer B.Cu) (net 2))
 (segment (start 119.327089 110.715255) (end 120.035529 110.006815) (width 0.25) (layer B.Cu) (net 2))
 (segment (start 108.784106 116.8146) (end 109.012126 116.58658) (width 0.25) (layer B.Cu) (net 2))
 (segment (start 109.012126 116.58658) (end 118.685915 116.58658) (width 0.25) (layer B.Cu) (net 2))
 (segment (start 120.035529 110.006815) (end 121.129731 110.006815) (width 0.25) (layer B.Cu) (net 2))
 (segment (start 121.129731 110.006815) (end 121.695416 110.006815) (width 0.25) (layer B.Cu) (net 2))
 (segment (start 122.85 110.6) (end 122.288601 110.6) (width 0.25) (layer F.Cu) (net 2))
 (segment (start 122.288601 110.6) (end 122.095415 110.406814) (width 0.25) (layer F.Cu) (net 2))
 (segment (start 122.095415 110.406814) (end 121.695416 110.006815) (width 0.25) (layer F.Cu) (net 2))
 (via (at 121.695416 110.006815) (size 0.8) (drill 0.4) (layers F.Cu B.Cu) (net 2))
 (segment (start 124.275 119.525) (end 124.275 119.025) (width 0.25) (layer F.Cu) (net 2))
 (segment (start 124.275 119.025) (end 124.199999 118.949999) (width 0.25) (layer F.Cu) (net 2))
 (segment (start 124.199999 118.949999) (end 122.971213 118.949999) (width 0.25) (layer F.Cu) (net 2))
 (segment (start 122.971213 118.949999) (end 122.046411 119.874801) (width 0.25) (layer F.Cu) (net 2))
 (segment (start 122.046411 119.874801) (end 108.646199 119.874801) (width 0.25) (layer F.Cu) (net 2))
 (segment (start 108.646199 119.874801) (end 107.251999 118.480601) (width 0.25) (layer F.Cu) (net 2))
 (segment (start 107.251999 118.480601) (end 107.251999 117.639601) (width 0.25) (layer F.Cu) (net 2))
 (segment (start 107.251999 117.639601) (end 107.577001 117.314599) (width 0.25) (layer F.Cu) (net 2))
 (segment (start 107.577001 117.314599) (end 108.077 116.8146) (width 0.25) (layer F.Cu) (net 2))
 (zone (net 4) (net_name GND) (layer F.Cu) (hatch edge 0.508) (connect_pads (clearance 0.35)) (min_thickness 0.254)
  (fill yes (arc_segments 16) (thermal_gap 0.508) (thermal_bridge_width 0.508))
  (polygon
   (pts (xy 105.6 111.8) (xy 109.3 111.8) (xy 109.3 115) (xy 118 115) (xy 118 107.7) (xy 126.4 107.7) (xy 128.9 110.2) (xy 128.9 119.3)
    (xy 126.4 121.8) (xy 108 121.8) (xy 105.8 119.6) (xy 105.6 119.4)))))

